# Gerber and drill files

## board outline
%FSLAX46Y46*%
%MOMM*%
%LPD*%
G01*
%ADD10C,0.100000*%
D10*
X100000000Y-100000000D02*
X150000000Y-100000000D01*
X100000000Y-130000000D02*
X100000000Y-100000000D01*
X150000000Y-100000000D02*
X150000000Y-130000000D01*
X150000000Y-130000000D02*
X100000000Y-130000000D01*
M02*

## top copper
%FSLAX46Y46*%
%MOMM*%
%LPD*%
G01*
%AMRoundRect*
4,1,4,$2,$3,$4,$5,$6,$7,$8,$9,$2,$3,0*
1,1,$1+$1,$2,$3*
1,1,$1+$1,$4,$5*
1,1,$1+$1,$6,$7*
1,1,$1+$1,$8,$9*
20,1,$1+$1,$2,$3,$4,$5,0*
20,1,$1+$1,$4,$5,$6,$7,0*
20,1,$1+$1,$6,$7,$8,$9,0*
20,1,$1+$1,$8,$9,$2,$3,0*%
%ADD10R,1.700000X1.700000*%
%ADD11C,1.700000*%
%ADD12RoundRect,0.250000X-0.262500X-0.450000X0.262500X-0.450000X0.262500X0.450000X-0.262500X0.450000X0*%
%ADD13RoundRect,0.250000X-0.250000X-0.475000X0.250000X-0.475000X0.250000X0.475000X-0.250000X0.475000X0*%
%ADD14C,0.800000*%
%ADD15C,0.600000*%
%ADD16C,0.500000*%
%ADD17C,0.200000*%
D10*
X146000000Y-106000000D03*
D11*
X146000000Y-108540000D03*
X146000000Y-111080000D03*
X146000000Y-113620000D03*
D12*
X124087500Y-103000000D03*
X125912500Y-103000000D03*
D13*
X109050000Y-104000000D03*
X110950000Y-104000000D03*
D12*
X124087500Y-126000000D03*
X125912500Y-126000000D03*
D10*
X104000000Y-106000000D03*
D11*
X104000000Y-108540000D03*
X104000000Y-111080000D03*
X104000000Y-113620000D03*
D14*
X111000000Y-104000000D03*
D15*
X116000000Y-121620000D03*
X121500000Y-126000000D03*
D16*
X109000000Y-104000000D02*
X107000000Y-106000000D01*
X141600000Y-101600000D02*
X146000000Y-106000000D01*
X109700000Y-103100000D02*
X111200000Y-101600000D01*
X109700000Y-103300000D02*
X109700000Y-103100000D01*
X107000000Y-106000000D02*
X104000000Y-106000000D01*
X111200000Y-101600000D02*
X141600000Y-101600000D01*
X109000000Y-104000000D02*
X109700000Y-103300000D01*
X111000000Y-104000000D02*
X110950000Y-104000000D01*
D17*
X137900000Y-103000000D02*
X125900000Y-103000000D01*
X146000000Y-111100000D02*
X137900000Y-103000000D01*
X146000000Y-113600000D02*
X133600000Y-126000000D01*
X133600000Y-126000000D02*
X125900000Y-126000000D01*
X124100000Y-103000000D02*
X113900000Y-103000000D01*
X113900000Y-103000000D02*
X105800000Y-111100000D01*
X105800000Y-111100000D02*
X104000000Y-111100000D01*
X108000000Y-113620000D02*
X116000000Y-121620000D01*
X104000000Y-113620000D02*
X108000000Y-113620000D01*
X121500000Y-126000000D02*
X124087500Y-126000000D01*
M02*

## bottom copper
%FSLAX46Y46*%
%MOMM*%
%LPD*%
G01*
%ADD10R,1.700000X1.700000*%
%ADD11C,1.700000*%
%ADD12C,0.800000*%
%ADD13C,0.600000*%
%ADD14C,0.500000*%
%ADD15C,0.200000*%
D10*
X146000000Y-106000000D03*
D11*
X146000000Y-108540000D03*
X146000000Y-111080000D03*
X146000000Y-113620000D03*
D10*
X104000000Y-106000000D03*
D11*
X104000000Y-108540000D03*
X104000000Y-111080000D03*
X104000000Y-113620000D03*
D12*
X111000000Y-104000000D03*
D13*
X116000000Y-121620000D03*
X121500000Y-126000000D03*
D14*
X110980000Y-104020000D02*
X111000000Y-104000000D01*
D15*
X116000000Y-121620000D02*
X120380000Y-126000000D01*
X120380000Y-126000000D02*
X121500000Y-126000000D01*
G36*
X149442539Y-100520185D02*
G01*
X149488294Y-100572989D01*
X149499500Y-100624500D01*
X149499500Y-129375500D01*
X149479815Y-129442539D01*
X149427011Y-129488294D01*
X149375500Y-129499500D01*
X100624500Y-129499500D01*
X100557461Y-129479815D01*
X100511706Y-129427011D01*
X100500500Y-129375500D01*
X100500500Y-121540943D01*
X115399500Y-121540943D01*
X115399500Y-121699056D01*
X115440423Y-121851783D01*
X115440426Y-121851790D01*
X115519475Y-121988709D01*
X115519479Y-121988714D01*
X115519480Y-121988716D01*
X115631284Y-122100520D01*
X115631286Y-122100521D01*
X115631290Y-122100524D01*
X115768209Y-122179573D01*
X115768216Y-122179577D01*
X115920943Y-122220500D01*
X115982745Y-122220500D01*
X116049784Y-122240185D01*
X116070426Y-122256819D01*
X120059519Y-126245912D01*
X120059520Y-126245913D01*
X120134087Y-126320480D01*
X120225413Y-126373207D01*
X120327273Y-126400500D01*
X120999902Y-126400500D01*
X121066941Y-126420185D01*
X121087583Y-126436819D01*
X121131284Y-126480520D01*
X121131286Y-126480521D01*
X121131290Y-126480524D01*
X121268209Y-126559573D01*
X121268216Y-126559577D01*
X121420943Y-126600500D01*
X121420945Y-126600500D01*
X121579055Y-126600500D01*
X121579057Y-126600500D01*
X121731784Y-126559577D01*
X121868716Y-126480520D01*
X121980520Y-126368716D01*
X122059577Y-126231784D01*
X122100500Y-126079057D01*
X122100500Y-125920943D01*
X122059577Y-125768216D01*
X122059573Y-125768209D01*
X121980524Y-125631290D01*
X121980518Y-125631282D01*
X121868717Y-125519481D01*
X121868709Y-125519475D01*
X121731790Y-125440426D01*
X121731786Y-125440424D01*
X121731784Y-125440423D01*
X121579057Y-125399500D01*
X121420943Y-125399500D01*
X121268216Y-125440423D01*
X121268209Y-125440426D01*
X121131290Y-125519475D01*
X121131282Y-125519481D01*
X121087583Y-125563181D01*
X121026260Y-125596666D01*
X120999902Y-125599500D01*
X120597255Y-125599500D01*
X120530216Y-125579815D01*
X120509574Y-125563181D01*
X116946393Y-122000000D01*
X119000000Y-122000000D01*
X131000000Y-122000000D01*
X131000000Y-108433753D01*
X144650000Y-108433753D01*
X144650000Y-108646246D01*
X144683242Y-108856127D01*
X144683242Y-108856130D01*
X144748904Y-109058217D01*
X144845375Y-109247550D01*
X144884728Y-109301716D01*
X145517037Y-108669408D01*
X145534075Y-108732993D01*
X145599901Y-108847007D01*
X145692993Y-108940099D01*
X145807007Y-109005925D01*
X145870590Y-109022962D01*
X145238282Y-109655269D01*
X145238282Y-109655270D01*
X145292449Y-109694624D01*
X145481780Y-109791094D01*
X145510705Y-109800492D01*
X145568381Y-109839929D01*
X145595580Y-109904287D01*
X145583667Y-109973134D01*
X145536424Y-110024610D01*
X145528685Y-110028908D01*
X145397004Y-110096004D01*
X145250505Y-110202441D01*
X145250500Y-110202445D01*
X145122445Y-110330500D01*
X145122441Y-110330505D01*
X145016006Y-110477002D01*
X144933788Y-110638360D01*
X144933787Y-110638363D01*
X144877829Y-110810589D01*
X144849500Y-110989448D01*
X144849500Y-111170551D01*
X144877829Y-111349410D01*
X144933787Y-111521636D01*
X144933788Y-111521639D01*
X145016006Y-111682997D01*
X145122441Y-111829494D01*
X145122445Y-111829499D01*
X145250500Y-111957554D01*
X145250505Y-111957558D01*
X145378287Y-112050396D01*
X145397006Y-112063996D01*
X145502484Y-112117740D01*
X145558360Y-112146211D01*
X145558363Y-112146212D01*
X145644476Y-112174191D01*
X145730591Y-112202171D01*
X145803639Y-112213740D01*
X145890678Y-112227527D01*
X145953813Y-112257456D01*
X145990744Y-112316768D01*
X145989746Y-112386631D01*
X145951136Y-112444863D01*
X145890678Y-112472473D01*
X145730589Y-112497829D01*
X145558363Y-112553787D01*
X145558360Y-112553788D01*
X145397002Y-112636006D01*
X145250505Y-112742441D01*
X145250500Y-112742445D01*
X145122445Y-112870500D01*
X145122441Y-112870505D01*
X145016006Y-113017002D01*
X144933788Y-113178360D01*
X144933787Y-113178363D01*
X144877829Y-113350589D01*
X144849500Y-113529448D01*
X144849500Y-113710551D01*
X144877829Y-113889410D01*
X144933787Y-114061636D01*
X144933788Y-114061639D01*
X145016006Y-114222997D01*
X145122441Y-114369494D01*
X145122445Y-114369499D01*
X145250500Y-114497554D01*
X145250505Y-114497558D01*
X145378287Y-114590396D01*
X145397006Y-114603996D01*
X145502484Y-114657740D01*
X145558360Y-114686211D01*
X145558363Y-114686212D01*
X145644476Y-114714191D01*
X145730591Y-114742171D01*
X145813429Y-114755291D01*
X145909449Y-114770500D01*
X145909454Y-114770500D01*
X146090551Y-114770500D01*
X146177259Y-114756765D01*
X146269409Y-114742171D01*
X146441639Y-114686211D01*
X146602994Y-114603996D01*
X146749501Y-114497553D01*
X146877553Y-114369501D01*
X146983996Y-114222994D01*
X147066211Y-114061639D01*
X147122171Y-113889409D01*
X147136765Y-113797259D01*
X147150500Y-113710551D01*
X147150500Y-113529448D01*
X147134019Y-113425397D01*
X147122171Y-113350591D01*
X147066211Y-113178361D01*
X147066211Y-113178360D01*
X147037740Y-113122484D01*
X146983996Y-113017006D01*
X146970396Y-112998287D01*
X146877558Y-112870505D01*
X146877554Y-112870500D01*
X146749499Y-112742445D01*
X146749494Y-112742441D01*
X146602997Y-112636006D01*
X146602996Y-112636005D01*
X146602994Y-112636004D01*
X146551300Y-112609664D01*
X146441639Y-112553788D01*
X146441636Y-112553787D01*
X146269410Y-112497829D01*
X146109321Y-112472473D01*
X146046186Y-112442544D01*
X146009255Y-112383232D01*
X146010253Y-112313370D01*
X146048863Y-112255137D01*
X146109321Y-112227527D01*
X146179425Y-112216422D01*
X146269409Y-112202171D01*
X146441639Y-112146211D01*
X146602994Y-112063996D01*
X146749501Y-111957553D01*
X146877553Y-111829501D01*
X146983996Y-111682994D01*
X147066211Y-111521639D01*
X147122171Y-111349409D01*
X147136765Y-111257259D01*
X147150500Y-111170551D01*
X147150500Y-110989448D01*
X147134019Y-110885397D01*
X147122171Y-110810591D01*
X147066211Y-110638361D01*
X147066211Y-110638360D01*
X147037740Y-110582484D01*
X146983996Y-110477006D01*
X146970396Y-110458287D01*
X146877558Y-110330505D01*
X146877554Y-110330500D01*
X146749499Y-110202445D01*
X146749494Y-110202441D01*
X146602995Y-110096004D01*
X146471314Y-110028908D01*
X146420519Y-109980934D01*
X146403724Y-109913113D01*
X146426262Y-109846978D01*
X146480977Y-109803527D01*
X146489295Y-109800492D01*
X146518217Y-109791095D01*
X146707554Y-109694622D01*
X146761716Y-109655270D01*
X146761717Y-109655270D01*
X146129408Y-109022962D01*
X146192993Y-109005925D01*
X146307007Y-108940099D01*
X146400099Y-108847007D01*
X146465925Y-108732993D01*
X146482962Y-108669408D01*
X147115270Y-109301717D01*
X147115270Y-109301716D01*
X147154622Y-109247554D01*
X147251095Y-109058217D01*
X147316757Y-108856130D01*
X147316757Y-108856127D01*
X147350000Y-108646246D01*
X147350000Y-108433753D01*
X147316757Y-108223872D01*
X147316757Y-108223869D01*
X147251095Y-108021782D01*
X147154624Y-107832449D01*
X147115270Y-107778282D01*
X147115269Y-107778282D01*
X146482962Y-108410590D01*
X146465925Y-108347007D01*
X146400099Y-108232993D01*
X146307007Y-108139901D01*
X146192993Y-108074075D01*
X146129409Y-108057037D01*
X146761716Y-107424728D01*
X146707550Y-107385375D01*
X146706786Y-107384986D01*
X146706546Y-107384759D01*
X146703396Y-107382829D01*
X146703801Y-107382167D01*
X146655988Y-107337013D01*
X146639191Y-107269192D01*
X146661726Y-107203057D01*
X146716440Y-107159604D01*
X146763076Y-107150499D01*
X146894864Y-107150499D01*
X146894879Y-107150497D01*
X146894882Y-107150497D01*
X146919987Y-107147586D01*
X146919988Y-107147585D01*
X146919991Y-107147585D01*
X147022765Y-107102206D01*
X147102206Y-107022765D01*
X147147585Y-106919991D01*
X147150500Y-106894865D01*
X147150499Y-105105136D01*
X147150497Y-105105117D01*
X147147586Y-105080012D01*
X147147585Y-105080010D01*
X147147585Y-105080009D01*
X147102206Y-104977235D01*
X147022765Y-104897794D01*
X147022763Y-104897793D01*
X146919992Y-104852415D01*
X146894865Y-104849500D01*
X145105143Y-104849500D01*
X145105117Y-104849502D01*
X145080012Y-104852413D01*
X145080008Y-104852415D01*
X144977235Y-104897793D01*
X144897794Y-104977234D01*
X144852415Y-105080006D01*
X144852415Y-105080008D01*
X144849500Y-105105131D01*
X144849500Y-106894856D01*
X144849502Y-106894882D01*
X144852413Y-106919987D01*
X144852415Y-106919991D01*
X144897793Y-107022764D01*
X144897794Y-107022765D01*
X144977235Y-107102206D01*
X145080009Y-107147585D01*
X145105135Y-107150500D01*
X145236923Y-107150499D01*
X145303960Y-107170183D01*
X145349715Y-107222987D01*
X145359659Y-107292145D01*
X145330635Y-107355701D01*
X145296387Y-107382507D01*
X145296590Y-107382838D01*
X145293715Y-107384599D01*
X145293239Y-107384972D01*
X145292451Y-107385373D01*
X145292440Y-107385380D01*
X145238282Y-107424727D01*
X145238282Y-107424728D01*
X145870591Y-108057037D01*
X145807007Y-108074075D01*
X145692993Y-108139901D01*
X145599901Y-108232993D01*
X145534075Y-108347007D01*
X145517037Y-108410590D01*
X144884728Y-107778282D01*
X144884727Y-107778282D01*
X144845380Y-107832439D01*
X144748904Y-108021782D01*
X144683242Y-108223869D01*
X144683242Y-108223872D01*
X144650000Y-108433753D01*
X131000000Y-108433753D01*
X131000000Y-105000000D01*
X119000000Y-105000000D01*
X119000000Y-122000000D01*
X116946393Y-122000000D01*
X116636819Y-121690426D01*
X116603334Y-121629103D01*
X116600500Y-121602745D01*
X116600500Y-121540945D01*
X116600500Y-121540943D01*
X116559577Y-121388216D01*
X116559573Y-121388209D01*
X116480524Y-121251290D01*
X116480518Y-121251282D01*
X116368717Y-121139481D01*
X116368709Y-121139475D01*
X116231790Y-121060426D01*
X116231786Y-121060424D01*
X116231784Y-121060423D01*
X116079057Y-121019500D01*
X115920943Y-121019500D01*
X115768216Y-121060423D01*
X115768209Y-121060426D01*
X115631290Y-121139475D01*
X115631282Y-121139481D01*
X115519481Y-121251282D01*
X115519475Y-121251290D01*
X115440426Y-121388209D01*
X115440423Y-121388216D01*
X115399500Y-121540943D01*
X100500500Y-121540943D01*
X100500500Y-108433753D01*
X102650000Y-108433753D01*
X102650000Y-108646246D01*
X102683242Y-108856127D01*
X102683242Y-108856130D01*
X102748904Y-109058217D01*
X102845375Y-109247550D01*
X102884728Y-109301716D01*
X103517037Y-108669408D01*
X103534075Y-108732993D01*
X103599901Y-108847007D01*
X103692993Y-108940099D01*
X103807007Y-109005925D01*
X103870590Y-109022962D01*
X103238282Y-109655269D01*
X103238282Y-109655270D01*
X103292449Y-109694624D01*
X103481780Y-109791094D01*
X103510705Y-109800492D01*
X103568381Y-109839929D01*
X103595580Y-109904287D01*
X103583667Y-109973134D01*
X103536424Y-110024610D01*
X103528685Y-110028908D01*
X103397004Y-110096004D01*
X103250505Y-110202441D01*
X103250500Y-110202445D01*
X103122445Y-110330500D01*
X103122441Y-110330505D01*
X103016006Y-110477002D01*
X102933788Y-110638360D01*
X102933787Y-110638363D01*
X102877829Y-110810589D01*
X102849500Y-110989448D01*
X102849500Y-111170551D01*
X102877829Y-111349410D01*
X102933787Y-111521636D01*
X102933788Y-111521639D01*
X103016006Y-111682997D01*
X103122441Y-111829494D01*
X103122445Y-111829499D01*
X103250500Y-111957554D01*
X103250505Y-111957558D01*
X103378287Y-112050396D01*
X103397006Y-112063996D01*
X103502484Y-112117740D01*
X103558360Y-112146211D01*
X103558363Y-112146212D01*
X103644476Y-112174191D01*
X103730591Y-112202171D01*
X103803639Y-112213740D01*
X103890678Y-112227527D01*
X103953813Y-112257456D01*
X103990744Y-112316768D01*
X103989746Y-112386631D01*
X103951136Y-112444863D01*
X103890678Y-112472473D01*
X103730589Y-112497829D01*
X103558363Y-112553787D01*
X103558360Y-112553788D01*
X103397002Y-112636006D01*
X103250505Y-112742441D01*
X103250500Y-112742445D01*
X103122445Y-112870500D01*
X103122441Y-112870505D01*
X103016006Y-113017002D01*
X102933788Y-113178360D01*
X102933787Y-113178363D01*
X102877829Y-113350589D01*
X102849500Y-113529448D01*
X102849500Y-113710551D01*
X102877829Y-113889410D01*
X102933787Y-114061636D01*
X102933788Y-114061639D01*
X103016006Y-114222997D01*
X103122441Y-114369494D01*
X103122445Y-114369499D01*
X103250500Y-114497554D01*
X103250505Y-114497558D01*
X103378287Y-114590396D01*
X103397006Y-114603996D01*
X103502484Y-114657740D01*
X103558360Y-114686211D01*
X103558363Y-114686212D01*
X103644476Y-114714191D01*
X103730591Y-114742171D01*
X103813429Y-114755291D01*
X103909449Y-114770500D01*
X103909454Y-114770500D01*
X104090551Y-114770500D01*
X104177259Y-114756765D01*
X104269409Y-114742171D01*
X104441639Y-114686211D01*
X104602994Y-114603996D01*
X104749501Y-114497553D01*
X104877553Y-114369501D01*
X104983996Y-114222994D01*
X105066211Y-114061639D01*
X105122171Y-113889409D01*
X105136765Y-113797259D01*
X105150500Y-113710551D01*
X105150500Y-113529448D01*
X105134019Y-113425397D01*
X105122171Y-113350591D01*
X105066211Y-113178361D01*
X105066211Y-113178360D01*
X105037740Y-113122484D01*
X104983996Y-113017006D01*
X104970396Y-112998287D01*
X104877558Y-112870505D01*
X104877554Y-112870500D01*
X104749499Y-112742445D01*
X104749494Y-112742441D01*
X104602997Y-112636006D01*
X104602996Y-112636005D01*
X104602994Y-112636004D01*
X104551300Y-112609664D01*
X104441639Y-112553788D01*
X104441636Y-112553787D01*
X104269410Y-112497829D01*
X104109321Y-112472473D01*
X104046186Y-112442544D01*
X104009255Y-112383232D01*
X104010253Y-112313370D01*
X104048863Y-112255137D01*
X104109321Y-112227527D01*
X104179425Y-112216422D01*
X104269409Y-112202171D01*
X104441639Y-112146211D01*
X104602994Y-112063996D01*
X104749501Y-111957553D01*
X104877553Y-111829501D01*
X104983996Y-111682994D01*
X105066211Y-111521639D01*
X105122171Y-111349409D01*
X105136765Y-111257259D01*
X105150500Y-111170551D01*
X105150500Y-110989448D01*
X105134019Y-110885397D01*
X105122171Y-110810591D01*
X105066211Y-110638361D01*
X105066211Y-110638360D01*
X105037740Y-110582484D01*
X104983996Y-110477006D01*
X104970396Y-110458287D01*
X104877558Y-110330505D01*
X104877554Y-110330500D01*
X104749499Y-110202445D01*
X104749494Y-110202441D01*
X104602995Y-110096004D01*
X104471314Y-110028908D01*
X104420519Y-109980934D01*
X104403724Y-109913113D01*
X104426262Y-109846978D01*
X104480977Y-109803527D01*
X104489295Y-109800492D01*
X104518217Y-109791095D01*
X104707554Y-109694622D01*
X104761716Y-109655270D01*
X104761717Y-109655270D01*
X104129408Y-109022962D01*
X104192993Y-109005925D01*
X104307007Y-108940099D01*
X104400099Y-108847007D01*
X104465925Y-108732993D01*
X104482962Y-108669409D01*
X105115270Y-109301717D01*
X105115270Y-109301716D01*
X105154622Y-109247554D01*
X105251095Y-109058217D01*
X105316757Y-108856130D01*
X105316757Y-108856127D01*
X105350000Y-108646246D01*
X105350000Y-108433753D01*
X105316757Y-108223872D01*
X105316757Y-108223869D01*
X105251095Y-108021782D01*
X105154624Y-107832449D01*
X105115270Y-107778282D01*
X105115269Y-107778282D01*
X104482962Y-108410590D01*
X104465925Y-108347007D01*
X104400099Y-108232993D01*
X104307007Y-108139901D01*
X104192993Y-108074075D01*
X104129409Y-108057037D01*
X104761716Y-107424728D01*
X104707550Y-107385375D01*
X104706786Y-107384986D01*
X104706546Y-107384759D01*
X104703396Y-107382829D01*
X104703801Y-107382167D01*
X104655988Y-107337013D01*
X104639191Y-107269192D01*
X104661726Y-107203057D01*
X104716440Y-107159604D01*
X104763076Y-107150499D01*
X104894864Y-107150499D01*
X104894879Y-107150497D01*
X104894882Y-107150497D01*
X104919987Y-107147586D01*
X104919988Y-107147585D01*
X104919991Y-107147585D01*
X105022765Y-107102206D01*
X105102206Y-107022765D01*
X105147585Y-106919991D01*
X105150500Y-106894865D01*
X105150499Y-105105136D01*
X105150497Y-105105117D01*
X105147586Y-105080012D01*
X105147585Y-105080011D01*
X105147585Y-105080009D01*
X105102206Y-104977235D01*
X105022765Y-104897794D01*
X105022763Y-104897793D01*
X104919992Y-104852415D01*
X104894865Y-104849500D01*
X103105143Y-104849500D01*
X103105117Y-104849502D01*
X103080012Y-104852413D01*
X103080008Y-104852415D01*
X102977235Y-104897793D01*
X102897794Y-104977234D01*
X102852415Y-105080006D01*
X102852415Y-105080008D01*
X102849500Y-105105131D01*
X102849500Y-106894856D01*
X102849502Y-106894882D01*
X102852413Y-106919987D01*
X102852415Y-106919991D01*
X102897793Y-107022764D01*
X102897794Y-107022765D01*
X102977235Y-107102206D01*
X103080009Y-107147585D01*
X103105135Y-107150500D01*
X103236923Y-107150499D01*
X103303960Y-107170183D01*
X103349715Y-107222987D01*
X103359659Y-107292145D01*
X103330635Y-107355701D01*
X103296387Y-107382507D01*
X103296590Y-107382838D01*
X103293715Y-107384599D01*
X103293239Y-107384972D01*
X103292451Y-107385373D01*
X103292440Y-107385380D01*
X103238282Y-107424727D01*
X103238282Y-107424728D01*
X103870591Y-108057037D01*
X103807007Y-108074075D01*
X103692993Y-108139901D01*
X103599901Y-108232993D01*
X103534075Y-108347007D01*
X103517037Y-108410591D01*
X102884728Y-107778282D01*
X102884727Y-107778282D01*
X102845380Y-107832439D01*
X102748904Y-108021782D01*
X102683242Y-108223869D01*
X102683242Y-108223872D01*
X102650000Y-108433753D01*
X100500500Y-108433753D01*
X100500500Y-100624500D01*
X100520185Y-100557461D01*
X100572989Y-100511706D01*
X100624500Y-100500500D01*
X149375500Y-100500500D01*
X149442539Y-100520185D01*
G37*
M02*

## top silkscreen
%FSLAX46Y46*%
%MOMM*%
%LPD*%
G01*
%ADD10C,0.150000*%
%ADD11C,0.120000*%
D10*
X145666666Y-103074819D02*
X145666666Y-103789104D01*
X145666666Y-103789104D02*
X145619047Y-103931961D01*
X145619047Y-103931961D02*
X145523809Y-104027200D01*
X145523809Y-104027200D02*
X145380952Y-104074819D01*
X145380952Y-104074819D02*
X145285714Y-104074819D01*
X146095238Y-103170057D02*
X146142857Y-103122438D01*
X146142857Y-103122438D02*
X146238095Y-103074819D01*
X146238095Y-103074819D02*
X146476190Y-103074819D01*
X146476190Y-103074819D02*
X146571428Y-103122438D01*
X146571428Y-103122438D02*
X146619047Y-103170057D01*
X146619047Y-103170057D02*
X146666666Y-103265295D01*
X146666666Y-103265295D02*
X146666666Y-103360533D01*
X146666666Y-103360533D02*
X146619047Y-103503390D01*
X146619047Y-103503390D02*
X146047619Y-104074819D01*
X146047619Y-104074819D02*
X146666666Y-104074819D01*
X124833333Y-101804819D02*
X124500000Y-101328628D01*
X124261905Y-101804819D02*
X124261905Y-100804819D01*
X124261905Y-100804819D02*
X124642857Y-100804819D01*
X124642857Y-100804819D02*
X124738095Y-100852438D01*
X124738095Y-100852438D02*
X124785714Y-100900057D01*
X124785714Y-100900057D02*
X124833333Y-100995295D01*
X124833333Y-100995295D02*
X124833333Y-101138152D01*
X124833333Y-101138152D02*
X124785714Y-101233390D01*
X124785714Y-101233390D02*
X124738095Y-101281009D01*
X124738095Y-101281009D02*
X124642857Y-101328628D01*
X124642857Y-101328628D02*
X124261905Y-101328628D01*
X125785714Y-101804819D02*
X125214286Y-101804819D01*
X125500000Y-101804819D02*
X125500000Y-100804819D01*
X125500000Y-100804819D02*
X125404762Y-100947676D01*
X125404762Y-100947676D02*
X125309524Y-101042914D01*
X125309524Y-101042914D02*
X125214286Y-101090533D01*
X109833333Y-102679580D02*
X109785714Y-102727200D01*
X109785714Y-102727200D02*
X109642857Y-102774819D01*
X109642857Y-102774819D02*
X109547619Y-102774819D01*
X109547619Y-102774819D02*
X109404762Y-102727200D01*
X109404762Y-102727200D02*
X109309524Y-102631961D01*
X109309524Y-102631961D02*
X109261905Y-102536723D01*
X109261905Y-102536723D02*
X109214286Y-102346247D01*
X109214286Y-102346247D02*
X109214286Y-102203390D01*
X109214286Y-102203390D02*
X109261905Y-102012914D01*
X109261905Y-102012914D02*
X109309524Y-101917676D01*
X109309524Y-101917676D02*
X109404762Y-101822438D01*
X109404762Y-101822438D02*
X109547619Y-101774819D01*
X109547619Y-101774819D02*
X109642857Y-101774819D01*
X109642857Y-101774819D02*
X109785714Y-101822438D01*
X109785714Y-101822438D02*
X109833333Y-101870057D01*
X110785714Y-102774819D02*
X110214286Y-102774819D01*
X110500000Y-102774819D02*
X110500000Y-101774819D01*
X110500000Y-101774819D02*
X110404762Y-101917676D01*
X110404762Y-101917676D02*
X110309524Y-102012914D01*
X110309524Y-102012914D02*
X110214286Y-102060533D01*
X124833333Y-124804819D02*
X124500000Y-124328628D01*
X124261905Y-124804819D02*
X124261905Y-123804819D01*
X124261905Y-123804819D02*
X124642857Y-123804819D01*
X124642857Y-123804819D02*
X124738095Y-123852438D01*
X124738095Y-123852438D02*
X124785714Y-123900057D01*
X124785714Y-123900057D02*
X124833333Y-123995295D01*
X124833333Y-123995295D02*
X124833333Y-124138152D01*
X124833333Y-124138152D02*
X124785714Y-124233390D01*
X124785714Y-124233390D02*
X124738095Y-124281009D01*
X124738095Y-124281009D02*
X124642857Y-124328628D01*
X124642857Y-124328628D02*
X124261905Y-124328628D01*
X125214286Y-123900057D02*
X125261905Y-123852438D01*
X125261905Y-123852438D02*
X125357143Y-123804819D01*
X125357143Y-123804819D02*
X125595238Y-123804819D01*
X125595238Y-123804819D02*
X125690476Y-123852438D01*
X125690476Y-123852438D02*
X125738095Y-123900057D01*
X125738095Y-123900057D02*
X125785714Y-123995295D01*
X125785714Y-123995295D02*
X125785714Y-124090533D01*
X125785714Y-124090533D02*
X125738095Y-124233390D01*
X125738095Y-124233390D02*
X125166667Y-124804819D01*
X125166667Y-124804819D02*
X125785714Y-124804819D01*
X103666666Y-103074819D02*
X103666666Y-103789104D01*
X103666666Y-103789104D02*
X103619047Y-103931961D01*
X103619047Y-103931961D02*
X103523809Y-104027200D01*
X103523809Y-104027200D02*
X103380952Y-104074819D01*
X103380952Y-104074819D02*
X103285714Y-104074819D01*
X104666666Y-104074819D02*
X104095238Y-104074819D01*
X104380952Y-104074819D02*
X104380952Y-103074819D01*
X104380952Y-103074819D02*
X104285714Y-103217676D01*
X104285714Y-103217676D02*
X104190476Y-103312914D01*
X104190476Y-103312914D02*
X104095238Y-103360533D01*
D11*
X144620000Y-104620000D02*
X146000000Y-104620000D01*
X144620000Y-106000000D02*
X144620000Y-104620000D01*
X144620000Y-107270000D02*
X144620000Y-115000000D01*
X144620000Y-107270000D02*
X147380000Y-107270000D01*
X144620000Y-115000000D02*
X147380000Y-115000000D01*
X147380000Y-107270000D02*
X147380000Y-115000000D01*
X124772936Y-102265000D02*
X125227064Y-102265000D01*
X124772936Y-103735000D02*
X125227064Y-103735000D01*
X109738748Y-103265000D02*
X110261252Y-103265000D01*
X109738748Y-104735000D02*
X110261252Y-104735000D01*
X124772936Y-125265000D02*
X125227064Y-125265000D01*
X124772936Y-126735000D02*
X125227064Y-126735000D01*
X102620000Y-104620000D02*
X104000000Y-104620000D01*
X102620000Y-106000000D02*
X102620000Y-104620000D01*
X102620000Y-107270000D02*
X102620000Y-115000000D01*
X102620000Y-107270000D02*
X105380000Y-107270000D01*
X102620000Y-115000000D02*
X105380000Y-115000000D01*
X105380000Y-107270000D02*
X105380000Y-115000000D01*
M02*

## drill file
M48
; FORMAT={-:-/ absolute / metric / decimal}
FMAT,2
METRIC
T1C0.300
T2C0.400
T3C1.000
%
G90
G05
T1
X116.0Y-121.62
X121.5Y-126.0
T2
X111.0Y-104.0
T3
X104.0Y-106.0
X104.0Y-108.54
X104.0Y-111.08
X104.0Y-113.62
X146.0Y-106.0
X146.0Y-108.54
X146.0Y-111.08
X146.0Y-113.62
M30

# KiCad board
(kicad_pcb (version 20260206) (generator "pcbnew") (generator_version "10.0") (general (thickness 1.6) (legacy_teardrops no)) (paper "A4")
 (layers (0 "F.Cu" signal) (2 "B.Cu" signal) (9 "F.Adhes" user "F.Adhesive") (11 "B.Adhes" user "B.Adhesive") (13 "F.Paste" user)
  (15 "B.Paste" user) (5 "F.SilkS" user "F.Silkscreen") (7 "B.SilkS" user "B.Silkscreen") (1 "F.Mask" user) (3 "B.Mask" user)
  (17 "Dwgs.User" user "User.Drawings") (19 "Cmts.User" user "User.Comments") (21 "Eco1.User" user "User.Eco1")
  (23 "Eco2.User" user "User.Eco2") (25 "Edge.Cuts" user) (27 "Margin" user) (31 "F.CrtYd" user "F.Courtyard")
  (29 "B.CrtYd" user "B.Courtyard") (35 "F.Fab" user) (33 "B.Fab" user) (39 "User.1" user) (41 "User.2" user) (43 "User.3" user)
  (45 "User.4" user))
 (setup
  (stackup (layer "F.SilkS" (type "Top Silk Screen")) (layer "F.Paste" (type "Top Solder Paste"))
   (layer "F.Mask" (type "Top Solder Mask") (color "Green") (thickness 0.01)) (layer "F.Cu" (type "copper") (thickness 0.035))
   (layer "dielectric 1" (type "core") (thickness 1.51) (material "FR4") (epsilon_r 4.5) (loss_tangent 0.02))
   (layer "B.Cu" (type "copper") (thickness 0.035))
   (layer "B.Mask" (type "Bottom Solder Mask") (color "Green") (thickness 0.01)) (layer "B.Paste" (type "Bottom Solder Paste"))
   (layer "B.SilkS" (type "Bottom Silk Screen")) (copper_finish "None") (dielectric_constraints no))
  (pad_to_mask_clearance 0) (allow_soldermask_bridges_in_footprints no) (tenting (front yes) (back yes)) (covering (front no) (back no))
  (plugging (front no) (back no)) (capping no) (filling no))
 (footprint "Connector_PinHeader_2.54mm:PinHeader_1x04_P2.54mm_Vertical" (layer "F.Cu") (at 146 106)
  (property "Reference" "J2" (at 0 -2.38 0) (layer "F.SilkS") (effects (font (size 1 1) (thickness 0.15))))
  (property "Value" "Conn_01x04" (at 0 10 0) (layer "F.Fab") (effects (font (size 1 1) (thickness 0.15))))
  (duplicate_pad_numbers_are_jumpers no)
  (fp_line (start -1.38 -1.38) (end 0 -1.38) (stroke (width 0.12) (type solid)) (layer "F.SilkS"))
  (fp_line (start -1.38 0) (end -1.38 -1.38) (stroke (width 0.12) (type solid)) (layer "F.SilkS"))
  (fp_line (start -1.38 1.27) (end -1.38 9) (stroke (width 0.12) (type solid)) (layer "F.SilkS"))
  (fp_line (start -1.38 1.27) (end 1.38 1.27) (stroke (width 0.12) (type solid)) (layer "F.SilkS"))
  (fp_line (start -1.38 9) (end 1.38 9) (stroke (width 0.12) (type solid)) (layer "F.SilkS"))
  (fp_line (start 1.38 1.27) (end 1.38 9) (stroke (width 0.12) (type solid)) (layer "F.SilkS"))
  (pad "1" thru_hole rect (at 0 0) (size 1.7 1.7) (drill 1) (layers "*.Cu" "*.Mask") (remove_unused_layers no) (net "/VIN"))
  (pad "2" thru_hole circle (at 0 2.54) (size 1.7 1.7) (drill 1) (layers "*.Cu" "*.Mask") (remove_unused_layers no) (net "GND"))
  (pad "3" thru_hole circle (at 0 5.08) (size 1.7 1.7) (drill 1) (layers "*.Cu" "*.Mask") (remove_unused_layers no) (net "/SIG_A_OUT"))
  (pad "4" thru_hole circle (at 0 7.62) (size 1.7 1.7) (drill 1) (layers "*.Cu" "*.Mask") (remove_unused_layers no) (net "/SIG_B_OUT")))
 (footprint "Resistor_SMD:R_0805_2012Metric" (layer "F.Cu") (at 125 103)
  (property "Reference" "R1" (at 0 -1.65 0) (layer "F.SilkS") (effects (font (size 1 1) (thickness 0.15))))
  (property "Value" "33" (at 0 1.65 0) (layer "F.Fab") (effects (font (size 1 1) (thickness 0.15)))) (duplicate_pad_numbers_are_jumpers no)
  (fp_line (start -0.227064 -0.735) (end 0.227064 -0.735) (stroke (width 0.12) (type solid)) (layer "F.SilkS"))
  (fp_line (start -0.227064 0.735) (end 0.227064 0.735) (stroke (width 0.12) (type solid)) (layer "F.SilkS"))
  (pad "1" smd roundrect (at -0.9125 0) (size 1.025 1.4) (layers "F.Cu" "F.Mask" "F.Paste") (roundrect_rratio 0.243902) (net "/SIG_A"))
  (pad "2" smd roundrect (at 0.9125 0) (size 1.025 1.4) (layers "F.Cu" "F.Mask" "F.Paste") (roundrect_rratio 0.243902) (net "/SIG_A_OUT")))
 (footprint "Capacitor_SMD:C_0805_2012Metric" (layer "F.Cu") (at 110 104)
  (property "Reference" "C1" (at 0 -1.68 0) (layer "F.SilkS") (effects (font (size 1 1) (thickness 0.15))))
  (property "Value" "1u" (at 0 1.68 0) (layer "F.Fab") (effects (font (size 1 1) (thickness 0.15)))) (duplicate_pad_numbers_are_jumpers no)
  (fp_line (start -0.261252 -0.735) (end 0.261252 -0.735) (stroke (width 0.12) (type solid)) (layer "F.SilkS"))
  (fp_line (start -0.261252 0.735) (end 0.261252 0.735) (stroke (width 0.12) (type solid)) (layer "F.SilkS"))
  (pad "1" smd roundrect (at -0.95 0) (size 1 1.45) (layers "F.Cu" "F.Mask" "F.Paste") (roundrect_rratio 0.25) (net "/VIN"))
  (pad "2" smd roundrect (at 0.95 0) (size 1 1.45) (layers "F.Cu" "F.Mask" "F.Paste") (roundrect_rratio 0.25) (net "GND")))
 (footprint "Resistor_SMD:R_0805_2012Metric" (layer "F.Cu") (at 125 126)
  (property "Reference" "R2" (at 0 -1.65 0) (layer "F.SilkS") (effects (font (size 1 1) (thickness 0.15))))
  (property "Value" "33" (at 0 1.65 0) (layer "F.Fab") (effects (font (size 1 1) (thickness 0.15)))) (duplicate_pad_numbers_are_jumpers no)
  (fp_line (start -0.227064 -0.735) (end 0.227064 -0.735) (stroke (width 0.12) (type solid)) (layer "F.SilkS"))
  (fp_line (start -0.227064 0.735) (end 0.227064 0.735) (stroke (width 0.12) (type solid)) (layer "F.SilkS"))
  (pad "1" smd roundrect (at -0.9125 0) (size 1.025 1.4) (layers "F.Cu" "F.Mask" "F.Paste") (roundrect_rratio 0.243902) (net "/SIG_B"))
  (pad "2" smd roundrect (at 0.9125 0) (size 1.025 1.4) (layers "F.Cu" "F.Mask" "F.Paste") (roundrect_rratio 0.243902) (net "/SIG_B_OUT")))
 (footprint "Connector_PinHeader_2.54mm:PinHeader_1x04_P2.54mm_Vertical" (layer "F.Cu") (at 104 106)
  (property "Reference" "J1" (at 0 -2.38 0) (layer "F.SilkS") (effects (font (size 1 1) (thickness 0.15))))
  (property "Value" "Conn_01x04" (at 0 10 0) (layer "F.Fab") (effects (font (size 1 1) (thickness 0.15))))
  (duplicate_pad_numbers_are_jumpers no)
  (fp_line (start -1.38 -1.38) (end 0 -1.38) (stroke (width 0.12) (type solid)) (layer "F.SilkS"))
  (fp_line (start -1.38 0) (end -1.38 -1.38) (stroke (width 0.12) (type solid)) (layer "F.SilkS"))
  (fp_line (start -1.38 1.27) (end -1.38 9) (stroke (width 0.12) (type solid)) (layer "F.SilkS"))
  (fp_line (start -1.38 1.27) (end 1.38 1.27) (stroke (width 0.12) (type solid)) (layer "F.SilkS"))
  (fp_line (start -1.38 9) (end 1.38 9) (stroke (width 0.12) (type solid)) (layer "F.SilkS"))
  (fp_line (start 1.38 1.27) (end 1.38 9) (stroke (width 0.12) (type solid)) (layer "F.SilkS"))
  (pad "1" thru_hole rect (at 0 0) (size 1.7 1.7) (drill 1) (layers "*.Cu" "*.Mask") (remove_unused_layers no) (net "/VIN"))
  (pad "2" thru_hole circle (at 0 2.54) (size 1.7 1.7) (drill 1) (layers "*.Cu" "*.Mask") (remove_unused_layers no) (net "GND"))
  (pad "3" thru_hole circle (at 0 5.08) (size 1.7 1.7) (drill 1) (layers "*.Cu" "*.Mask") (remove_unused_layers no) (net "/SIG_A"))
  (pad "4" thru_hole circle (at 0 7.62) (size 1.7 1.7) (drill 1) (layers "*.Cu" "*.Mask") (remove_unused_layers no) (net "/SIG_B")))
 (gr_line (start 100 100) (end 150 100) (stroke (width 0.1) (type default)) (layer "Edge.Cuts"))
 (gr_line (start 100 130) (end 100 100) (stroke (width 0.1) (type default)) (layer "Edge.Cuts"))
 (gr_line (start 150 100) (end 150 130) (stroke (width 0.1) (type default)) (layer "Edge.Cuts"))
 (gr_line (start 150 130) (end 100 130) (stroke (width 0.1) (type default)) (layer "Edge.Cuts"))
 (segment (start 109 104) (end 107 106) (width 0.5) (layer "F.Cu") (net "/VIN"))
 (segment (start 141.6 101.6) (end 146 106) (width 0.5) (layer "F.Cu") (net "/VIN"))
 (segment (start 109.7 103.1) (end 111.2 101.6) (width 0.5) (layer "F.Cu") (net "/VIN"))
 (segment (start 109.7 103.3) (end 109.7 103.1) (width 0.5) (layer "F.Cu") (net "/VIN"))
 (segment (start 107 106) (end 104 106) (width 0.5) (layer "F.Cu") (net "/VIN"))
 (segment (start 111.2 101.6) (end 141.6 101.6) (width 0.5) (layer "F.Cu") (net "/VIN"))
 (segment (start 109 104) (end 109.7 103.3) (width 0.5) (layer "F.Cu") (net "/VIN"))
 (segment (start 111 104) (end 110.95 104) (width 0.5) (layer "F.Cu") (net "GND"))
 (via (at 111 104) (size 0.8) (drill 0.4) (layers "F.Cu" "B.Cu") (capping yes) (filling yes) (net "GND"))
 (segment (start 110.98 104.02) (end 111 104) (width 0.5) (layer "B.Cu") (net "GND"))
 (segment (start 137.9 103) (end 125.9 103) (width 0.2) (layer "F.Cu") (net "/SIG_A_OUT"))
 (segment (start 146 111.1) (end 137.9 103) (width 0.2) (layer "F.Cu") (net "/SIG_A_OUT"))
 (segment (start 146 113.6) (end 133.6 126) (width 0.2) (layer "F.Cu") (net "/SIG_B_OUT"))
 (segment (start 133.6 126) (end 125.9 126) (width 0.2) (layer "F.Cu") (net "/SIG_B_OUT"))
 (segment (start 124.1 103) (end 113.9 103) (width 0.2) (layer "F.Cu") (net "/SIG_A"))
 (segment (start 113.9 103) (end 105.8 111.1) (width 0.2) (layer "F.Cu") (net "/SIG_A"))
 (segment (start 105.8 111.1) (end 104 111.1) (width 0.2) (layer "F.Cu") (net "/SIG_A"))
 (segment (start 108 113.62) (end 116 121.62) (width 0.2) (locked yes) (layer "F.Cu") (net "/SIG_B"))
 (segment (start 104 113.62) (end 108 113.62) (width 0.2) (locked yes) (layer "F.Cu") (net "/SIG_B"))
 (segment (start 121.5 126) (end 124.0875 126) (width 0.2) (locked yes) (layer "F.Cu") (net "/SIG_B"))
 (via (at 116 121.62) (size 0.6) (drill 0.3) (layers "F.Cu" "B.Cu") (locked yes) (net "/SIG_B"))
 (via (at 121.5 126) (size 0.6) (drill 0.3) (layers "F.Cu" "B.Cu") (locked yes) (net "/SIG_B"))
 (segment (start 116 121.62) (end 120.38 126) (width 0.2) (locked yes) (layer "B.Cu") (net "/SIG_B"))
 (segment (start 120.38 126) (end 121.5 126) (width 0.2) (locked yes) (layer "B.Cu") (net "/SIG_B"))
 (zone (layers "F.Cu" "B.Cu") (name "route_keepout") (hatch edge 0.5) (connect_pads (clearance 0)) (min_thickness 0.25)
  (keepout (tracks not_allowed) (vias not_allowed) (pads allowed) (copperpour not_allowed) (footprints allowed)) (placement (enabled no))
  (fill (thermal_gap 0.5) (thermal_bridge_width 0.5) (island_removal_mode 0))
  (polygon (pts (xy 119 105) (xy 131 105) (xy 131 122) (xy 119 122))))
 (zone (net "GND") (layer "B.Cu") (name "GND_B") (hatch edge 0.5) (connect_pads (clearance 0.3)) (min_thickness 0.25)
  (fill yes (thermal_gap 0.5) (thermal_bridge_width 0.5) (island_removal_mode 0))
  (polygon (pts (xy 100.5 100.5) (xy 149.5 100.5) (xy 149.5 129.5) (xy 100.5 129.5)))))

